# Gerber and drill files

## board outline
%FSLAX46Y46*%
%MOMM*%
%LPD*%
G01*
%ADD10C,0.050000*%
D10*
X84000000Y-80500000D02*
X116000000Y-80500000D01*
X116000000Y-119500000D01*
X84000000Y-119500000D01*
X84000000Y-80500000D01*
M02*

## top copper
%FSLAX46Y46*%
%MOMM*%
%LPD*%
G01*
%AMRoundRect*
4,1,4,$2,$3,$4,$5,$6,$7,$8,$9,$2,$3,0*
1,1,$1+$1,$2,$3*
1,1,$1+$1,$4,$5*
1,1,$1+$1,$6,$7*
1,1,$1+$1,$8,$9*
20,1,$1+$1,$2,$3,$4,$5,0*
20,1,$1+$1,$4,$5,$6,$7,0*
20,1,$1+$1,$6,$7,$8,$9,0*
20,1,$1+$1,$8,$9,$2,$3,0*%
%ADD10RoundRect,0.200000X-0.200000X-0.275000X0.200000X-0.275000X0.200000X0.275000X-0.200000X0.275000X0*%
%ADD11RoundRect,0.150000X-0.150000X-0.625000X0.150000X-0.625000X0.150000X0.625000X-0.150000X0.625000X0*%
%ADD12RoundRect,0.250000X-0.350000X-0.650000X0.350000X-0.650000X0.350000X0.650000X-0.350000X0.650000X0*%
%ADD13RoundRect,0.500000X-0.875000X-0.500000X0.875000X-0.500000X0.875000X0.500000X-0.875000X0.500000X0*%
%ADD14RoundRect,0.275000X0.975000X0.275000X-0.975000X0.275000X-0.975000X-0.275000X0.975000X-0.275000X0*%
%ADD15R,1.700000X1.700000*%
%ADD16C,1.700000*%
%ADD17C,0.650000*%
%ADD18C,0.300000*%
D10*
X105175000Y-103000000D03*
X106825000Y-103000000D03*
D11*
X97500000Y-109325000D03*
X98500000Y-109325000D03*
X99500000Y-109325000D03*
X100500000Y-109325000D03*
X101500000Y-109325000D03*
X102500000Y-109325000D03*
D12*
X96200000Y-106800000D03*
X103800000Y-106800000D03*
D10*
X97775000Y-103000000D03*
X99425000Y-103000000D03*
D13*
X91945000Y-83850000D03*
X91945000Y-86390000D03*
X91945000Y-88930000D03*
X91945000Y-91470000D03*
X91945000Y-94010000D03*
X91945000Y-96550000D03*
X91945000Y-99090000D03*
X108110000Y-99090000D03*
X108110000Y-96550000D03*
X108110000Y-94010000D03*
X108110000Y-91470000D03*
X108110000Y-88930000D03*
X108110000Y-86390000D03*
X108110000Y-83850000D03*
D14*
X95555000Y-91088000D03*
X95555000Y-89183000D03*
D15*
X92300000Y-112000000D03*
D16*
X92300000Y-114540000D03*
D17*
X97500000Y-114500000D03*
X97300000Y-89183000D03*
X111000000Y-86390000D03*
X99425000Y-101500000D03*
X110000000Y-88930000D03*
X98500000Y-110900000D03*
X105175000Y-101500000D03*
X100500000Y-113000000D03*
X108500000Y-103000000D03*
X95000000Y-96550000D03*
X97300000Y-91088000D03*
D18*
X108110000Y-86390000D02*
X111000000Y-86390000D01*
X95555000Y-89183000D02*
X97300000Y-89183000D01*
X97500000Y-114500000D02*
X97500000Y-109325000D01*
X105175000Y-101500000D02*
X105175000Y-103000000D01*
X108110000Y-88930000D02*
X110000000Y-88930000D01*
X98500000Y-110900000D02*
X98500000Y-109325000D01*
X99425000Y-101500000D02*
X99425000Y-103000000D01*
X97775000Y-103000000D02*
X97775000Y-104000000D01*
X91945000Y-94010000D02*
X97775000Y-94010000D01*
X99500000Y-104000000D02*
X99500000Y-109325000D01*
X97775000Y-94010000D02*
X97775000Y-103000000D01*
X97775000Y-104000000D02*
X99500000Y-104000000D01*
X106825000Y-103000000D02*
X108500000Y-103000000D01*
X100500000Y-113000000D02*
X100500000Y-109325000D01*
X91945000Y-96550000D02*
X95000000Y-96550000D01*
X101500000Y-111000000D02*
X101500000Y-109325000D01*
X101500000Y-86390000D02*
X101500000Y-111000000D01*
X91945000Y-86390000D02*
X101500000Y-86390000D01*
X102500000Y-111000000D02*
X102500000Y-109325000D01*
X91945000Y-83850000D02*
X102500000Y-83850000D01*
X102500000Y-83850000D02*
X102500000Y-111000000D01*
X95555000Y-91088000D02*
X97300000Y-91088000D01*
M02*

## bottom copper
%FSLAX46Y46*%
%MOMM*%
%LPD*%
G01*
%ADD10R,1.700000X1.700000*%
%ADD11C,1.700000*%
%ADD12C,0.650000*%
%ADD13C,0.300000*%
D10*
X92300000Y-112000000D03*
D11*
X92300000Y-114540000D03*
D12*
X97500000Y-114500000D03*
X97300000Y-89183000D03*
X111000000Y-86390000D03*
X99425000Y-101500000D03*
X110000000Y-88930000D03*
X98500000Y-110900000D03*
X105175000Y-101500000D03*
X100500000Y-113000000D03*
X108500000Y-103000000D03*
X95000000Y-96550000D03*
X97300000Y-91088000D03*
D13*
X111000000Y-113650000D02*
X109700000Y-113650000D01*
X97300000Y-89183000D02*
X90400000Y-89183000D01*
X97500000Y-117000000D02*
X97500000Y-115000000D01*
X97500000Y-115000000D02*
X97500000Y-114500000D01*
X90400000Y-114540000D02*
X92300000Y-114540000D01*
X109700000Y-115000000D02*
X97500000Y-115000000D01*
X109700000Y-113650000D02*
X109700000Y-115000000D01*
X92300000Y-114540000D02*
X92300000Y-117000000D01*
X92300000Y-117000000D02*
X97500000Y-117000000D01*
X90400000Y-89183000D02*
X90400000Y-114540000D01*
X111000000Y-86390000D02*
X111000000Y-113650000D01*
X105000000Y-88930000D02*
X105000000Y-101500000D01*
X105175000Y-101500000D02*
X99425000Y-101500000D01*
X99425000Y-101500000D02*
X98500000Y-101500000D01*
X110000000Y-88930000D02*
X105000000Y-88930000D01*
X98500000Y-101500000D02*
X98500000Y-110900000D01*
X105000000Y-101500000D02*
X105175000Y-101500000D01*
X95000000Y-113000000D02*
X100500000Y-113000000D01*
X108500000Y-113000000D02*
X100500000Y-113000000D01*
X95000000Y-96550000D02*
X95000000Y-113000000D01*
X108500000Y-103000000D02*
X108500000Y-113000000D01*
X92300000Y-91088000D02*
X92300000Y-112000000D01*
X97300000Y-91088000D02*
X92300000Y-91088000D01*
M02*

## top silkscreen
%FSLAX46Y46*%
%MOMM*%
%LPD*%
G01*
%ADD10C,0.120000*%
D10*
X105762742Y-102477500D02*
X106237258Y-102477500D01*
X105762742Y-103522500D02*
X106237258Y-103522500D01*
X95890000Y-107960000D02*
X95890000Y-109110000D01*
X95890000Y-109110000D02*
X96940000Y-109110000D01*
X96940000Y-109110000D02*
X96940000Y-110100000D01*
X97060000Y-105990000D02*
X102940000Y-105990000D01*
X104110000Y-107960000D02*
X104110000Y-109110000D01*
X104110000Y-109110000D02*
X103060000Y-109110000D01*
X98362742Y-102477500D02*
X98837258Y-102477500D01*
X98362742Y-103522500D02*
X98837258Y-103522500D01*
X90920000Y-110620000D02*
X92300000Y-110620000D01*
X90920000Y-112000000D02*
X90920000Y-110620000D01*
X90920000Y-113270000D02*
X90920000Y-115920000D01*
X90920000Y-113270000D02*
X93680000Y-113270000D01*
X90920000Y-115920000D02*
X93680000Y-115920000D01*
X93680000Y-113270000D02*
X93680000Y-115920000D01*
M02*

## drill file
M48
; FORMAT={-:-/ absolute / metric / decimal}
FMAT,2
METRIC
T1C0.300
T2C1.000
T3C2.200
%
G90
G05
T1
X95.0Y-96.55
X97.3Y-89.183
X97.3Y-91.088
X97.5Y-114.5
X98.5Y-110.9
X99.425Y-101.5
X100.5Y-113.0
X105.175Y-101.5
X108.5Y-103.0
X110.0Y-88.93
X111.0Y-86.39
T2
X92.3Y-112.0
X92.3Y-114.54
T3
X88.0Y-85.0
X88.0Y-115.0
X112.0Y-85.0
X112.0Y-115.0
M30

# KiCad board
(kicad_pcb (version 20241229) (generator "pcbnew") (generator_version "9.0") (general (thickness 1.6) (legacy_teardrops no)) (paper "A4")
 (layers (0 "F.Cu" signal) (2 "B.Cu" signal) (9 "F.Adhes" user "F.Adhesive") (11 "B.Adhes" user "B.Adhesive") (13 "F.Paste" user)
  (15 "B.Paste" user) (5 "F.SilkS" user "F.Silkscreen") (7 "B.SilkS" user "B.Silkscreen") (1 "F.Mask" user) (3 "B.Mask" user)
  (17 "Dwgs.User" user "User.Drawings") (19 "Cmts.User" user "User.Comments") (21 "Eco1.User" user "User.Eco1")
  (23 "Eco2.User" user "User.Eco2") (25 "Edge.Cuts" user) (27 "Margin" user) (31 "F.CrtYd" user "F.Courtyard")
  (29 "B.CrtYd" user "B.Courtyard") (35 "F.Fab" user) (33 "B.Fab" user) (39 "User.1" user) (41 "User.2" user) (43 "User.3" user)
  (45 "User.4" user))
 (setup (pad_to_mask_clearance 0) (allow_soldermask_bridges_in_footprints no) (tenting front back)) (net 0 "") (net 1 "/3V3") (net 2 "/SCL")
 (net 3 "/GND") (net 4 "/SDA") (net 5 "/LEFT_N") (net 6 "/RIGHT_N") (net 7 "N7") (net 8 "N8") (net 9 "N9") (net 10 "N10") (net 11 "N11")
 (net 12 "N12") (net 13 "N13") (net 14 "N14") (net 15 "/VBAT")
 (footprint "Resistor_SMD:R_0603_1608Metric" (layer "F.Cu") (at 106 103)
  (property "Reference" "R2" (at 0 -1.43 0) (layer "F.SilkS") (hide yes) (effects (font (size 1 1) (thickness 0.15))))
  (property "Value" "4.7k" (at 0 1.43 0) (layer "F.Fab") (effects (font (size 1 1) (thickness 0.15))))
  (fp_line (start -0.237258 -0.5225) (end 0.237258 -0.5225) (stroke (width 0.12) (type solid)) (layer "F.SilkS"))
  (fp_line (start -0.237258 0.5225) (end 0.237258 0.5225) (stroke (width 0.12) (type solid)) (layer "F.SilkS"))
  (pad "1" smd roundrect (at -0.825 0) (size 0.8 0.95) (layers "F.Cu" "F.Mask" "F.Paste") (roundrect_rratio 0.25) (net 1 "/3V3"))
  (pad "2" smd roundrect (at 0.825 0) (size 0.8 0.95) (layers "F.Cu" "F.Mask" "F.Paste") (roundrect_rratio 0.25) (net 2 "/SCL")))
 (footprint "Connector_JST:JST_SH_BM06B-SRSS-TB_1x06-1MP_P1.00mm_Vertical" (layer "F.Cu") (at 100 108)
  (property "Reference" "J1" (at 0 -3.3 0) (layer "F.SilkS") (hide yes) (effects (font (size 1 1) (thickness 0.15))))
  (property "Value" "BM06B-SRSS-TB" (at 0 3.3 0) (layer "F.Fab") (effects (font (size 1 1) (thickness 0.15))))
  (fp_line (start -4.11 -0.04) (end -4.11 1.11) (stroke (width 0.12) (type solid)) (layer "F.SilkS"))
  (fp_line (start -4.11 1.11) (end -3.06 1.11) (stroke (width 0.12) (type solid)) (layer "F.SilkS"))
  (fp_line (start -3.06 1.11) (end -3.06 2.1) (stroke (width 0.12) (type solid)) (layer "F.SilkS"))
  (fp_line (start -2.94 -2.01) (end 2.94 -2.01) (stroke (width 0.12) (type solid)) (layer "F.SilkS"))
  (fp_line (start 4.11 -0.04) (end 4.11 1.11) (stroke (width 0.12) (type solid)) (layer "F.SilkS"))
  (fp_line (start 4.11 1.11) (end 3.06 1.11) (stroke (width 0.12) (type solid)) (layer "F.SilkS"))
  (pad "1" smd roundrect (at -2.5 1.325) (size 0.6 1.55) (layers "F.Cu" "F.Mask" "F.Paste") (roundrect_rratio 0.25) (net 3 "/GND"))
  (pad "2" smd roundrect (at -1.5 1.325) (size 0.6 1.55) (layers "F.Cu" "F.Mask" "F.Paste") (roundrect_rratio 0.25) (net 1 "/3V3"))
  (pad "3" smd roundrect (at -0.5 1.325) (size 0.6 1.55) (layers "F.Cu" "F.Mask" "F.Paste") (roundrect_rratio 0.25) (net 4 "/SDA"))
  (pad "4" smd roundrect (at 0.5 1.325) (size 0.6 1.55) (layers "F.Cu" "F.Mask" "F.Paste") (roundrect_rratio 0.25) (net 2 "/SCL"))
  (pad "5" smd roundrect (at 1.5 1.325) (size 0.6 1.55) (layers "F.Cu" "F.Mask" "F.Paste") (roundrect_rratio 0.25) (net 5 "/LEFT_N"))
  (pad "6" smd roundrect (at 2.5 1.325) (size 0.6 1.55) (layers "F.Cu" "F.Mask" "F.Paste") (roundrect_rratio 0.25) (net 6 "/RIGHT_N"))
  (pad "MP" smd roundrect (at -3.8 -1.2) (size 1.2 1.8) (layers "F.Cu" "F.Mask" "F.Paste") (roundrect_rratio 0.208333))
  (pad "MP" smd roundrect (at 3.8 -1.2) (size 1.2 1.8) (layers "F.Cu" "F.Mask" "F.Paste") (roundrect_rratio 0.208333)))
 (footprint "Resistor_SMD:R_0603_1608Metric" (layer "F.Cu") (at 98.6 103)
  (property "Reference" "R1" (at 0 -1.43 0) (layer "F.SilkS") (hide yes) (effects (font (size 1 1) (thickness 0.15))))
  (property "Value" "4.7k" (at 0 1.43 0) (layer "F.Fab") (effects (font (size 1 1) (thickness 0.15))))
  (fp_line (start -0.237258 -0.5225) (end 0.237258 -0.5225) (stroke (width 0.12) (type solid)) (layer "F.SilkS"))
  (fp_line (start -0.237258 0.5225) (end 0.237258 0.5225) (stroke (width 0.12) (type solid)) (layer "F.SilkS"))
  (pad "1" smd roundrect (at -0.825 0) (size 0.8 0.95) (layers "F.Cu" "F.Mask" "F.Paste") (roundrect_rratio 0.25) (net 4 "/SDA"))
  (pad "2" smd roundrect (at 0.825 0) (size 0.8 0.95) (layers "F.Cu" "F.Mask" "F.Paste") (roundrect_rratio 0.25) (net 1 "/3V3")))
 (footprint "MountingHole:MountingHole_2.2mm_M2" (layer "F.Cu") (at 112 115)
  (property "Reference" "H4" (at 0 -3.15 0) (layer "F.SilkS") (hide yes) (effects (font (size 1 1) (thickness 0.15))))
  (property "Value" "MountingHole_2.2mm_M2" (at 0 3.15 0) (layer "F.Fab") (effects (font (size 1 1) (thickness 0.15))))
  (pad "" np_thru_hole circle (at 0 0) (size 2.2 2.2) (drill 2.2) (layers "*.Cu" "*.Mask")))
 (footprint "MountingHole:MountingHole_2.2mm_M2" (layer "F.Cu") (at 112 85)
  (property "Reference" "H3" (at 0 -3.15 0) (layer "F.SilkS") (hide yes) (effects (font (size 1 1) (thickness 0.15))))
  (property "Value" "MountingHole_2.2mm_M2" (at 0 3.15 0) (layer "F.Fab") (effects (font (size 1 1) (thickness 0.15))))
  (pad "" np_thru_hole circle (at 0 0) (size 2.2 2.2) (drill 2.2) (layers "*.Cu" "*.Mask")))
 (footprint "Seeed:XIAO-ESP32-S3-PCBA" (layer "F.Cu") (at 91.11 101.97)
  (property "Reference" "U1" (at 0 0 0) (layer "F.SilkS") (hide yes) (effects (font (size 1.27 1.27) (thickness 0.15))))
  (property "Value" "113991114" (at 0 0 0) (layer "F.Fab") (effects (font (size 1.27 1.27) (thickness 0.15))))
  (pad "1" smd roundrect (at 0.835 -18.12) (size 2.75 2) (layers "F.Cu" "F.Mask" "F.Paste") (roundrect_rratio 0.25) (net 6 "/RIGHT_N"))
  (pad "2" smd roundrect (at 0.835 -15.58) (size 2.75 2) (layers "F.Cu" "F.Mask" "F.Paste") (roundrect_rratio 0.25) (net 5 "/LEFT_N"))
  (pad "3" smd roundrect (at 0.835 -13.04) (size 2.75 2) (layers "F.Cu" "F.Mask" "F.Paste") (roundrect_rratio 0.25) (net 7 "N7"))
  (pad "4" smd roundrect (at 0.835 -10.5) (size 2.75 2) (layers "F.Cu" "F.Mask" "F.Paste") (roundrect_rratio 0.25) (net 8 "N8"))
  (pad "5" smd roundrect (at 0.835 -7.96) (size 2.75 2) (layers "F.Cu" "F.Mask" "F.Paste") (roundrect_rratio 0.25) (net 4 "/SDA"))
  (pad "6" smd roundrect (at 0.835 -5.42) (size 2.75 2) (layers "F.Cu" "F.Mask" "F.Paste") (roundrect_rratio 0.25) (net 2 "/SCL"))
  (pad "7" smd roundrect (at 0.835 -2.88) (size 2.75 2) (layers "F.Cu" "F.Mask" "F.Paste") (roundrect_rratio 0.25) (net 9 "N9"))
  (pad "8" smd roundrect (at 17 -2.88) (size 2.75 2) (layers "F.Cu" "F.Mask" "F.Paste") (roundrect_rratio 0.25) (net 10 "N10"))
  (pad "9" smd roundrect (at 17 -5.42) (size 2.75 2) (layers "F.Cu" "F.Mask" "F.Paste") (roundrect_rratio 0.25) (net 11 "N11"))
  (pad "10" smd roundrect (at 17 -7.96) (size 2.75 2) (layers "F.Cu" "F.Mask" "F.Paste") (roundrect_rratio 0.25) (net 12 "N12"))
  (pad "11" smd roundrect (at 17 -10.5) (size 2.75 2) (layers "F.Cu" "F.Mask" "F.Paste") (roundrect_rratio 0.25) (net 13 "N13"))
  (pad "12" smd roundrect (at 17 -13.04) (size 2.75 2) (layers "F.Cu" "F.Mask" "F.Paste") (roundrect_rratio 0.25) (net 1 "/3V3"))
  (pad "13" smd roundrect (at 17 -15.58) (size 2.75 2) (layers "F.Cu" "F.Mask" "F.Paste") (roundrect_rratio 0.25) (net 3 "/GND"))
  (pad "14" smd roundrect (at 17 -18.12) (size 2.75 2) (layers "F.Cu" "F.Mask" "F.Paste") (roundrect_rratio 0.25) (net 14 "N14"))
  (pad "15" smd roundrect (at 4.445 -10.882 180) (size 2.5 1.1) (layers "F.Cu" "F.Mask" "F.Paste") (roundrect_rratio 0.25) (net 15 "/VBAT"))
  (pad "16" smd roundrect (at 4.445 -12.787 180) (size 2.5 1.1) (layers "F.Cu" "F.Mask" "F.Paste") (roundrect_rratio 0.25) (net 3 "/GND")))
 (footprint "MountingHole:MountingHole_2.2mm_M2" (layer "F.Cu") (at 88 85)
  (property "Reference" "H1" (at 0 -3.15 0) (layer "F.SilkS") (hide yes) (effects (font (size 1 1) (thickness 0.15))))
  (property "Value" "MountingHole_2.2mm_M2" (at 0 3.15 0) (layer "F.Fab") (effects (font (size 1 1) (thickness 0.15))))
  (pad "" np_thru_hole circle (at 0 0) (size 2.2 2.2) (drill 2.2) (layers "*.Cu" "*.Mask")))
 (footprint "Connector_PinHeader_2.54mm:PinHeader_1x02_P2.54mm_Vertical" (layer "F.Cu") (at 92.3 112)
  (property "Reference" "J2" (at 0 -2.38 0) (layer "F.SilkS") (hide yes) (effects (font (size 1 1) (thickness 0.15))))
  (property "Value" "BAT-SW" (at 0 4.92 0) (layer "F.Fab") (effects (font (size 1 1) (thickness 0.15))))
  (fp_line (start -1.38 -1.38) (end 0 -1.38) (stroke (width 0.12) (type solid)) (layer "F.SilkS"))
  (fp_line (start -1.38 0) (end -1.38 -1.38) (stroke (width 0.12) (type solid)) (layer "F.SilkS"))
  (fp_line (start -1.38 1.27) (end -1.38 3.92) (stroke (width 0.12) (type solid)) (layer "F.SilkS"))
  (fp_line (start -1.38 1.27) (end 1.38 1.27) (stroke (width 0.12) (type solid)) (layer "F.SilkS"))
  (fp_line (start -1.38 3.92) (end 1.38 3.92) (stroke (width 0.12) (type solid)) (layer "F.SilkS"))
  (fp_line (start 1.38 1.27) (end 1.38 3.92) (stroke (width 0.12) (type solid)) (layer "F.SilkS"))
  (pad "1" thru_hole rect (at 0 0) (size 1.7 1.7) (drill 1) (layers "*.Cu" "*.Mask") (remove_unused_layers no) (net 15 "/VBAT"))
  (pad "2" thru_hole circle (at 0 2.54) (size 1.7 1.7) (drill 1) (layers "*.Cu" "*.Mask") (remove_unused_layers no) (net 3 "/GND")))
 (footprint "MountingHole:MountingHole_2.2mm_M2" (layer "F.Cu") (at 88 115)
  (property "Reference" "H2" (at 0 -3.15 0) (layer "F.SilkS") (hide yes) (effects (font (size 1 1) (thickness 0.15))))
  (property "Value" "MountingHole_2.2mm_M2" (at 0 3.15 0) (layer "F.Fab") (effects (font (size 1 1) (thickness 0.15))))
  (pad "" np_thru_hole circle (at 0 0) (size 2.2 2.2) (drill 2.2) (layers "*.Cu" "*.Mask")))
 (gr_rect (start 84 80.5) (end 116 119.5) (stroke (width 0.05) (type default)) (fill no) (layer "Edge.Cuts"))
 (segment (start 108.11 86.39) (end 111 86.39) (width 0.3) (layer "F.Cu") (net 3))
 (segment (start 95.555 89.183) (end 97.3 89.183) (width 0.3) (layer "F.Cu") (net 3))
 (segment (start 97.5 114.5) (end 97.5 109.325) (width 0.3) (layer "F.Cu") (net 3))
 (via (at 97.5 114.5) (size 0.65) (drill 0.3) (layers "F.Cu" "B.Cu") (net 3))
 (via (at 97.3 89.183) (size 0.65) (drill 0.3) (layers "F.Cu" "B.Cu") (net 3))
 (via (at 111 86.39) (size 0.65) (drill 0.3) (layers "F.Cu" "B.Cu") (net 3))
 (segment (start 111 113.65) (end 109.7 113.65) (width 0.3) (layer "B.Cu") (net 3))
 (segment (start 97.3 89.183) (end 90.4 89.183) (width 0.3) (layer "B.Cu") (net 3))
 (segment (start 97.5 117) (end 97.5 115) (width 0.3) (layer "B.Cu") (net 3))
 (segment (start 97.5 115) (end 97.5 114.5) (width 0.3) (layer "B.Cu") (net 3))
 (segment (start 90.4 114.54) (end 92.3 114.54) (width 0.3) (layer "B.Cu") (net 3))
 (segment (start 109.7 115) (end 97.5 115) (width 0.3) (layer "B.Cu") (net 3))
 (segment (start 109.7 113.65) (end 109.7 115) (width 0.3) (layer "B.Cu") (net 3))
 (segment (start 92.3 114.54) (end 92.3 117) (width 0.3) (layer "B.Cu") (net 3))
 (segment (start 92.3 117) (end 97.5 117) (width 0.3) (layer "B.Cu") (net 3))
 (segment (start 90.4 89.183) (end 90.4 114.54) (width 0.3) (layer "B.Cu") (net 3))
 (segment (start 111 86.39) (end 111 113.65) (width 0.3) (layer "B.Cu") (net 3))
 (segment (start 105.175 101.5) (end 105.175 103) (width 0.3) (layer "F.Cu") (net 1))
 (segment (start 108.11 88.93) (end 110 88.93) (width 0.3) (layer "F.Cu") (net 1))
 (segment (start 98.5 110.9) (end 98.5 109.325) (width 0.3) (layer "F.Cu") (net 1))
 (segment (start 99.425 101.5) (end 99.425 103) (width 0.3) (layer "F.Cu") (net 1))
 (via (at 99.425 101.5) (size 0.65) (drill 0.3) (layers "F.Cu" "B.Cu") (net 1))
 (via (at 110 88.93) (size 0.65) (drill 0.3) (layers "F.Cu" "B.Cu") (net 1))
 (via (at 98.5 110.9) (size 0.65) (drill 0.3) (layers "F.Cu" "B.Cu") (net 1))
 (via (at 105.175 101.5) (size 0.65) (drill 0.3) (layers "F.Cu" "B.Cu") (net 1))
 (segment (start 105 88.93) (end 105 101.5) (width 0.3) (layer "B.Cu") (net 1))
 (segment (start 105.175 101.5) (end 99.425 101.5) (width 0.3) (layer "B.Cu") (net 1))
 (segment (start 99.425 101.5) (end 98.5 101.5) (width 0.3) (layer "B.Cu") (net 1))
 (segment (start 110 88.93) (end 105 88.93) (width 0.3) (layer "B.Cu") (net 1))
 (segment (start 98.5 101.5) (end 98.5 110.9) (width 0.3) (layer "B.Cu") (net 1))
 (segment (start 105 101.5) (end 105.175 101.5) (width 0.3) (layer "B.Cu") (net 1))
 (segment (start 97.775 103) (end 97.775 104) (width 0.3) (layer "F.Cu") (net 4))
 (segment (start 91.945 94.01) (end 97.775 94.01) (width 0.3) (layer "F.Cu") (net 4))
 (segment (start 99.5 104) (end 99.5 109.325) (width 0.3) (layer "F.Cu") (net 4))
 (segment (start 97.775 94.01) (end 97.775 103) (width 0.3) (layer "F.Cu") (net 4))
 (segment (start 97.775 104) (end 99.5 104) (width 0.3) (layer "F.Cu") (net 4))
 (segment (start 106.825 103) (end 108.5 103) (width 0.3) (layer "F.Cu") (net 2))
 (segment (start 100.5 113) (end 100.5 109.325) (width 0.3) (layer "F.Cu") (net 2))
 (segment (start 91.945 96.55) (end 95 96.55) (width 0.3) (layer "F.Cu") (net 2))
 (via (at 100.5 113) (size 0.65) (drill 0.3) (layers "F.Cu" "B.Cu") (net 2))
 (via (at 108.5 103) (size 0.65) (drill 0.3) (layers "F.Cu" "B.Cu") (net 2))
 (via (at 95 96.55) (size 0.65) (drill 0.3) (layers "F.Cu" "B.Cu") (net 2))
 (segment (start 95 113) (end 100.5 113) (width 0.3) (layer "B.Cu") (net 2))
 (segment (start 108.5 113) (end 100.5 113) (width 0.3) (layer "B.Cu") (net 2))
 (segment (start 95 96.55) (end 95 113) (width 0.3) (layer "B.Cu") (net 2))
 (segment (start 108.5 103) (end 108.5 113) (width 0.3) (layer "B.Cu") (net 2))
 (segment (start 101.5 111) (end 101.5 109.325) (width 0.3) (layer "F.Cu") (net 5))
 (segment (start 101.5 86.39) (end 101.5 111) (width 0.3) (layer "F.Cu") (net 5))
 (segment (start 91.945 86.39) (end 101.5 86.39) (width 0.3) (layer "F.Cu") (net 5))
 (segment (start 102.5 111) (end 102.5 109.325) (width 0.3) (layer "F.Cu") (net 6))
 (segment (start 91.945 83.85) (end 102.5 83.85) (width 0.3) (layer "F.Cu") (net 6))
 (segment (start 102.5 83.85) (end 102.5 111) (width 0.3) (layer "F.Cu") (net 6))
 (segment (start 95.555 91.088) (end 97.3 91.088) (width 0.3) (layer "F.Cu") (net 15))
 (via (at 97.3 91.088) (size 0.65) (drill 0.3) (layers "F.Cu" "B.Cu") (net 15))
 (segment (start 92.3 91.088) (end 92.3 112) (width 0.3) (layer "B.Cu") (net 15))
 (segment (start 97.3 91.088) (end 92.3 91.088) (width 0.3) (layer "B.Cu") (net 15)))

